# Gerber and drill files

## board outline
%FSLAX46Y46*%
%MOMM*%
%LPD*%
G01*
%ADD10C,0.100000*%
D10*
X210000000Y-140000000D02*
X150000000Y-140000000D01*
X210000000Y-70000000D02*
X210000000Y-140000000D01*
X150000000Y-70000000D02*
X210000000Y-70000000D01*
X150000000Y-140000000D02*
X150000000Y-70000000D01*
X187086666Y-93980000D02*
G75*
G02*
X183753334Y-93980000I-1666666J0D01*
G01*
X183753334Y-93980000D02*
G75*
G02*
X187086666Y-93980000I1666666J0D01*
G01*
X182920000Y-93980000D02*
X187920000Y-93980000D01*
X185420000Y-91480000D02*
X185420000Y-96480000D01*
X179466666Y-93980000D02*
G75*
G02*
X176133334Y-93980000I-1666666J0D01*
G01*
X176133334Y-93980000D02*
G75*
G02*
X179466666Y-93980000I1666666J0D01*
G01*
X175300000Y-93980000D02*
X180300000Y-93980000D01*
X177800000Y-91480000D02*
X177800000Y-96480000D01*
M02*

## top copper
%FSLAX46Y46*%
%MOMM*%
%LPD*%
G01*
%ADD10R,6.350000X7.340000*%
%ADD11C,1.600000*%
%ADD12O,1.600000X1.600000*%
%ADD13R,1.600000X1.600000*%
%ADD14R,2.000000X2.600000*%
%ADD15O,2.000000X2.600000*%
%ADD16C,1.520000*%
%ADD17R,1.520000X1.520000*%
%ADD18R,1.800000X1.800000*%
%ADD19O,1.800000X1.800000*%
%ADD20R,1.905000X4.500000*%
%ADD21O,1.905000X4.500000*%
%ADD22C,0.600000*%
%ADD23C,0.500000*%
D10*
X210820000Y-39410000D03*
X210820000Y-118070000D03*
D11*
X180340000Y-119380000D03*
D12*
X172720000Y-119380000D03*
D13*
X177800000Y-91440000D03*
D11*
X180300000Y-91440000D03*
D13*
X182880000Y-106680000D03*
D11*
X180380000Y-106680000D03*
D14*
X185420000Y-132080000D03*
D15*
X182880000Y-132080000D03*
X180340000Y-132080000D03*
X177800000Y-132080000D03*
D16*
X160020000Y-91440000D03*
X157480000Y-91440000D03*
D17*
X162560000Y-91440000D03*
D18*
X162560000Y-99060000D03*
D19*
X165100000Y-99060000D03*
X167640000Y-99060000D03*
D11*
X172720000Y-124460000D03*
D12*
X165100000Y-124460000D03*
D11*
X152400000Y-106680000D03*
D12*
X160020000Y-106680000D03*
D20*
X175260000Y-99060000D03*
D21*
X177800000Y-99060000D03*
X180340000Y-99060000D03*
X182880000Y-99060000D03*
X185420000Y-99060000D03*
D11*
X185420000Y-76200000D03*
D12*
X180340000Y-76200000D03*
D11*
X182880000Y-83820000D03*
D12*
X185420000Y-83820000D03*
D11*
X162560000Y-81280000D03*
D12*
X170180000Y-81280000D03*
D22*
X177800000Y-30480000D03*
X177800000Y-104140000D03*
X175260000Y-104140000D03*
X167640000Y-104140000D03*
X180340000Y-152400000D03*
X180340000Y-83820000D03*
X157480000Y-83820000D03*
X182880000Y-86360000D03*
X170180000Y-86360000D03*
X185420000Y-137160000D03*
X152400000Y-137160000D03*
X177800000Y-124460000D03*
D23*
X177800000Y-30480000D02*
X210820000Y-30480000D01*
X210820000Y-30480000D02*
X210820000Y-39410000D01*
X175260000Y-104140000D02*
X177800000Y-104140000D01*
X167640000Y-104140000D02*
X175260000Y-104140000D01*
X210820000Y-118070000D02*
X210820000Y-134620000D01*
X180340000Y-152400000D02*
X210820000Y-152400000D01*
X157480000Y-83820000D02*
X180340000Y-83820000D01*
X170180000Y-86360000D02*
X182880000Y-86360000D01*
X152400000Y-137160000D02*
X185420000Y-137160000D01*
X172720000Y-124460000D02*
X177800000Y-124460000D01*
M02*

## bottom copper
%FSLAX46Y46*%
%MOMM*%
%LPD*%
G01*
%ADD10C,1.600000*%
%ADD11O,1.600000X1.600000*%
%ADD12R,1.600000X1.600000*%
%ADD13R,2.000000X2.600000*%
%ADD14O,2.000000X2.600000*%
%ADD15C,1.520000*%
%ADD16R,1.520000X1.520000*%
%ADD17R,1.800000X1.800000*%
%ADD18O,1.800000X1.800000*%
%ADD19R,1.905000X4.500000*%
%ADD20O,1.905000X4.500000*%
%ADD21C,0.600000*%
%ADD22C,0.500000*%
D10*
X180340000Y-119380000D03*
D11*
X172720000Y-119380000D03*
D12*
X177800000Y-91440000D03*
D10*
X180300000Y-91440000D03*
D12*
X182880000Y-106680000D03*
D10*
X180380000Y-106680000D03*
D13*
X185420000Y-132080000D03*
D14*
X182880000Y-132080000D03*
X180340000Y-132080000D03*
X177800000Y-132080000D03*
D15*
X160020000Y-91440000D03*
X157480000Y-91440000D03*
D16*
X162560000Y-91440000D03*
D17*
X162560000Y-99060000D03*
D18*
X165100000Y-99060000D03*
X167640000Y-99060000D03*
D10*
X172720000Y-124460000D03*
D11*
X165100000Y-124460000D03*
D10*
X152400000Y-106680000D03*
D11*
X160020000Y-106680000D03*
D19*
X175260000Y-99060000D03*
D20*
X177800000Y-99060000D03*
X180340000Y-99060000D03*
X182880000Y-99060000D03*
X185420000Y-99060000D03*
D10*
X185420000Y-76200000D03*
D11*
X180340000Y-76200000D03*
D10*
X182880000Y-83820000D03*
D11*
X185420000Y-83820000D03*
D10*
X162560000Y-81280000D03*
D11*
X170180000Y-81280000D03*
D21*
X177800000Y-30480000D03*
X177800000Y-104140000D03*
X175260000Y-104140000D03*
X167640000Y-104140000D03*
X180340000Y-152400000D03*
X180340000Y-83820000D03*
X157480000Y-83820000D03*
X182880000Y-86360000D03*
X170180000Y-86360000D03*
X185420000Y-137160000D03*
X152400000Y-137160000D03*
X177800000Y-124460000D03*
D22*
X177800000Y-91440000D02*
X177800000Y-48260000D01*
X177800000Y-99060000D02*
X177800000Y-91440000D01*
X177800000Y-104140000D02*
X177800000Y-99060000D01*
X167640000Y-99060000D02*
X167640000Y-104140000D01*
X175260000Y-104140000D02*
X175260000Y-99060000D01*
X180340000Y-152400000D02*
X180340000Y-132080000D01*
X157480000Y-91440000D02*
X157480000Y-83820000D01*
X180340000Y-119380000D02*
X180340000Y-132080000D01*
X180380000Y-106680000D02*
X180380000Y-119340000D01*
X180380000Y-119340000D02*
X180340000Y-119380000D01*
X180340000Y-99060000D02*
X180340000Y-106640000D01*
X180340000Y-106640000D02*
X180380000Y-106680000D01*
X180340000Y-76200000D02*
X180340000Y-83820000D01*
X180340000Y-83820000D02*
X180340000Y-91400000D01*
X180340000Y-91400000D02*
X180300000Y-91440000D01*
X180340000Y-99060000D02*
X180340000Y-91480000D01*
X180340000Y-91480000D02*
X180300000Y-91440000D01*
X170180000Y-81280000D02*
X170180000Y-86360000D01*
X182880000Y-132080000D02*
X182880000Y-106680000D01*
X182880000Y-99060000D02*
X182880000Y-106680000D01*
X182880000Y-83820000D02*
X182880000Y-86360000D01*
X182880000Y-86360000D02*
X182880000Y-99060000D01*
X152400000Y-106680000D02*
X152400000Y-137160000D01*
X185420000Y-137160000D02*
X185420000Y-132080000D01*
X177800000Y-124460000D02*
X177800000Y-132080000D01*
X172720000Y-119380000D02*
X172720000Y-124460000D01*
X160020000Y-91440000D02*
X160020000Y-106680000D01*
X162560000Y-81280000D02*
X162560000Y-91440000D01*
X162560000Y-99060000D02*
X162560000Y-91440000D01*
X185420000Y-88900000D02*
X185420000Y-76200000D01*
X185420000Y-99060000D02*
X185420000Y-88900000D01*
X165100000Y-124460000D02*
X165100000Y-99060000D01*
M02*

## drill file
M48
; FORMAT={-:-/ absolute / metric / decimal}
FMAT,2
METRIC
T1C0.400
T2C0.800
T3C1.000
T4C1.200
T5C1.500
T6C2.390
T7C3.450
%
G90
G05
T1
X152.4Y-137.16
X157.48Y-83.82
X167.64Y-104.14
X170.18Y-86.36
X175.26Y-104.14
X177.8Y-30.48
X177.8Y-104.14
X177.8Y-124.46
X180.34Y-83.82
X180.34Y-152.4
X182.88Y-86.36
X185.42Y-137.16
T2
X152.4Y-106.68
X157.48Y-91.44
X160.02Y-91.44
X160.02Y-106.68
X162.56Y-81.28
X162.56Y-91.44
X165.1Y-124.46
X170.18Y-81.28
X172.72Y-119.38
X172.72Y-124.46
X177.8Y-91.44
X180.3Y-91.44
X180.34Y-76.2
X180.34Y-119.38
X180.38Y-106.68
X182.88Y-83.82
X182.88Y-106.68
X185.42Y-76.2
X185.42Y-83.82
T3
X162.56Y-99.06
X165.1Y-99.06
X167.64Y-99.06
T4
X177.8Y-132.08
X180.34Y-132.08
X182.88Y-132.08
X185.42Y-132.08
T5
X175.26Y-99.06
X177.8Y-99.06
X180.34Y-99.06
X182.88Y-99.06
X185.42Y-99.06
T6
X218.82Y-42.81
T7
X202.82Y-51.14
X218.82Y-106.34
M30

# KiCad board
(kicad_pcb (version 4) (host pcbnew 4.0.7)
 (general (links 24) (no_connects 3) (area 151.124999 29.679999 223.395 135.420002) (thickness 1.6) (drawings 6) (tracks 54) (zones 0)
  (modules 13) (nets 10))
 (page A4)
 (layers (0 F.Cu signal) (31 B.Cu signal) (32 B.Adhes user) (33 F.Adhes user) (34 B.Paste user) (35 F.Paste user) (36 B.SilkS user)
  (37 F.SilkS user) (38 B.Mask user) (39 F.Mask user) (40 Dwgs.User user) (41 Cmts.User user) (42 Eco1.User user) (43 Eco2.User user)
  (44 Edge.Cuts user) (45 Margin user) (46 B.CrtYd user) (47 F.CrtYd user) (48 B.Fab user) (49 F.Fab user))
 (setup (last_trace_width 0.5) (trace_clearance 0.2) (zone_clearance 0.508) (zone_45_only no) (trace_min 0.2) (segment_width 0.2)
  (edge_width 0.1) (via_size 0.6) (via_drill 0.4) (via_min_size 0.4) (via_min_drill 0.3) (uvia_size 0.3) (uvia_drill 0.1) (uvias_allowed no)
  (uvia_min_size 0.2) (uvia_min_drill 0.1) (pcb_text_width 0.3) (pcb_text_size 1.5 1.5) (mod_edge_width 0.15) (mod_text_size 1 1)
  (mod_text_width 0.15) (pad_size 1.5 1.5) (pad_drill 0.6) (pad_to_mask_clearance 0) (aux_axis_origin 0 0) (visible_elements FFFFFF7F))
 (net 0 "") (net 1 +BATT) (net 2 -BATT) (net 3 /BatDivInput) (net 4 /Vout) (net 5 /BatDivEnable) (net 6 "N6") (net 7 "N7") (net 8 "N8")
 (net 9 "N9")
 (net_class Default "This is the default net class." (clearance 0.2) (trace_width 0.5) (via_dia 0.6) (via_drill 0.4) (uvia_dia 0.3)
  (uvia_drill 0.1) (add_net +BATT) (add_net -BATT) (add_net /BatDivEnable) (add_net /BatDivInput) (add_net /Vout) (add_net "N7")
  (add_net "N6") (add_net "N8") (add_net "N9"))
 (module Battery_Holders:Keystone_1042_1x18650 (layer F.Cu) (at 210.82 78.74 270)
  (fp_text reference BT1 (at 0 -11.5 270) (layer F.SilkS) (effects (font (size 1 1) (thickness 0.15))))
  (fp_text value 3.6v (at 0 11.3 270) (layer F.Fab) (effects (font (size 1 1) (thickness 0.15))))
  (pad 1 smd rect (at -39.33 0 270) (size 7.34 6.35) (layers F.Cu F.Paste F.Mask) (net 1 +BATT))
  (pad 2 smd rect (at 39.33 0 270) (size 7.34 6.35) (layers F.Cu F.Paste F.Mask) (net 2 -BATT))
  (pad "" np_thru_hole circle (at 27.6 -8 270) (size 3.45 3.45) (drill 3.45) (layers *.Cu *.Mask))
  (pad "" np_thru_hole circle (at -27.6 8 270) (size 3.45 3.45) (drill 3.45) (layers *.Cu *.Mask))
  (pad "" np_thru_hole circle (at -35.93 -8 270) (size 2.39 2.39) (drill 2.39) (layers *.Cu *.Mask)))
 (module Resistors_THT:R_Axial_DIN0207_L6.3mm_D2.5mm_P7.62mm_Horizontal (layer F.Cu) (at 180.34 119.38 180)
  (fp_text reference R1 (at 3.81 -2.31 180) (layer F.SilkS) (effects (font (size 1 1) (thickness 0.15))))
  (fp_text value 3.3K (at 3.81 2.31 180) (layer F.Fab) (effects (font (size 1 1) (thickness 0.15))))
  (pad 1 thru_hole circle (at 0 0 180) (size 1.6 1.6) (drill 0.8) (layers *.Cu *.Mask) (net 2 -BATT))
  (pad 2 thru_hole oval (at 7.62 0 180) (size 1.6 1.6) (drill 0.8) (layers *.Cu *.Mask) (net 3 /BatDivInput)))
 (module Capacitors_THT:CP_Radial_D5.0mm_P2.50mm (layer F.Cu) (at 177.8 91.44)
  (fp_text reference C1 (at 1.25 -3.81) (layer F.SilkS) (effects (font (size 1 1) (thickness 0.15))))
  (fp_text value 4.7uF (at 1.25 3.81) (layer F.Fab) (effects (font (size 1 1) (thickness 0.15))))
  (pad 1 thru_hole rect (at 0 0) (size 1.6 1.6) (drill 0.8) (layers *.Cu *.Mask) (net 1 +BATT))
  (pad 2 thru_hole circle (at 2.5 0) (size 1.6 1.6) (drill 0.8) (layers *.Cu *.Mask) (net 2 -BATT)))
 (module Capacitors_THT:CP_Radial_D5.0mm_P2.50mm (layer F.Cu) (at 182.88 106.68 180)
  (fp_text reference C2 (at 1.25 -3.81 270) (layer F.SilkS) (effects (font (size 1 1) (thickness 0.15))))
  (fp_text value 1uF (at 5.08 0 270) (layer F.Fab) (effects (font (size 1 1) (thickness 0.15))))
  (pad 1 thru_hole rect (at 0 0 180) (size 1.6 1.6) (drill 0.8) (layers *.Cu *.Mask) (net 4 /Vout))
  (pad 2 thru_hole circle (at 2.5 0 180) (size 1.6 1.6) (drill 0.8) (layers *.Cu *.Mask) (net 2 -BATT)))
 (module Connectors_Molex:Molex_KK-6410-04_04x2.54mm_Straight (layer F.Cu) (at 185.42 132.08 180)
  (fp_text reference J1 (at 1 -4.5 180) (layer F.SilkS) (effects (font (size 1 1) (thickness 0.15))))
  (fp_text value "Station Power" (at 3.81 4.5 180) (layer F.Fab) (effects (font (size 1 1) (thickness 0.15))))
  (pad 1 thru_hole rect (at 0 0 180) (size 2 2.6) (drill 1.2) (layers *.Cu *.Mask) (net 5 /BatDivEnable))
  (pad 2 thru_hole oval (at 2.54 0 180) (size 2 2.6) (drill 1.2) (layers *.Cu *.Mask) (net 4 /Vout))
  (pad 3 thru_hole oval (at 5.08 0 180) (size 2 2.6) (drill 1.2) (layers *.Cu *.Mask) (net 2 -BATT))
  (pad 4 thru_hole oval (at 7.62 0 180) (size 2 2.6) (drill 1.2) (layers *.Cu *.Mask) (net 3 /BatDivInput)))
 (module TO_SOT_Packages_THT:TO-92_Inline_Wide (layer F.Cu) (at 162.56 91.44 180)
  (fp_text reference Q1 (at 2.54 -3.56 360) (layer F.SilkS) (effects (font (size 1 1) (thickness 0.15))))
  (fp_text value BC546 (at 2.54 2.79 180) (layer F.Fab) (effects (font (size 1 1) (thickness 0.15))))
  (pad 2 thru_hole circle (at 2.54 0 270) (size 1.52 1.52) (drill 0.8) (layers *.Cu *.Mask) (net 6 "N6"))
  (pad 3 thru_hole circle (at 5.08 0 270) (size 1.52 1.52) (drill 0.8) (layers *.Cu *.Mask) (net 2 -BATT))
  (pad 1 thru_hole rect (at 0 0 270) (size 1.52 1.52) (drill 0.8) (layers *.Cu *.Mask) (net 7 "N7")))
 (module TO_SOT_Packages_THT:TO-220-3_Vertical (layer F.Cu) (at 162.56 99.06)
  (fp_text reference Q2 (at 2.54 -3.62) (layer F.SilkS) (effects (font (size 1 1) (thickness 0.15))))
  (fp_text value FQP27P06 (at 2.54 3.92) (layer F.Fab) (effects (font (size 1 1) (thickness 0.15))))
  (pad 1 thru_hole rect (at 0 0) (size 1.8 1.8) (drill 1) (layers *.Cu *.Mask) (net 7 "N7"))
  (pad 2 thru_hole oval (at 2.54 0) (size 1.8 1.8) (drill 1) (layers *.Cu *.Mask) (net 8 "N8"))
  (pad 3 thru_hole oval (at 5.08 0) (size 1.8 1.8) (drill 1) (layers *.Cu *.Mask) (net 1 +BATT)))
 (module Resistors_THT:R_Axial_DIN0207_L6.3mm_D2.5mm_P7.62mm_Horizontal (layer F.Cu) (at 172.72 124.46 180)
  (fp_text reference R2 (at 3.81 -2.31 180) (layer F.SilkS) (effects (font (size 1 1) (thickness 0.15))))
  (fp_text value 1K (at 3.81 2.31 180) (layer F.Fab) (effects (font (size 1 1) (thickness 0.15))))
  (pad 1 thru_hole circle (at 0 0 180) (size 1.6 1.6) (drill 0.8) (layers *.Cu *.Mask) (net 3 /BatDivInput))
  (pad 2 thru_hole oval (at 7.62 0 180) (size 1.6 1.6) (drill 0.8) (layers *.Cu *.Mask) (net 8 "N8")))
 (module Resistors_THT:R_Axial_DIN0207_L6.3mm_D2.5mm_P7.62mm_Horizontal (layer F.Cu) (at 152.4 106.68)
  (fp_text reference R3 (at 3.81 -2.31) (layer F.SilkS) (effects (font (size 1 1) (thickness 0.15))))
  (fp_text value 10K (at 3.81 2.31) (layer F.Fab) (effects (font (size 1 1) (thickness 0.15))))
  (pad 1 thru_hole circle (at 0 0) (size 1.6 1.6) (drill 0.8) (layers *.Cu *.Mask) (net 5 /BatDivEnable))
  (pad 2 thru_hole oval (at 7.62 0) (size 1.6 1.6) (drill 0.8) (layers *.Cu *.Mask) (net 6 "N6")))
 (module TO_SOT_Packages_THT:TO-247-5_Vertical (layer F.Cu) (at 175.26 99.06)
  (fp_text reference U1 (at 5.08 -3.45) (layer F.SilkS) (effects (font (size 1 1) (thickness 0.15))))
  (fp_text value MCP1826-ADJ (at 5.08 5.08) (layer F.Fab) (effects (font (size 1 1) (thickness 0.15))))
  (pad 1 thru_hole rect (at 0 0) (size 1.905 4.5) (drill 1.5) (layers *.Cu *.Mask) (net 1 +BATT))
  (pad 2 thru_hole oval (at 2.54 0) (size 1.905 4.5) (drill 1.5) (layers *.Cu *.Mask) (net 1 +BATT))
  (pad 3 thru_hole oval (at 5.08 0) (size 1.905 4.5) (drill 1.5) (layers *.Cu *.Mask) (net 2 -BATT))
  (pad 4 thru_hole oval (at 7.62 0) (size 1.905 4.5) (drill 1.5) (layers *.Cu *.Mask) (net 4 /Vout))
  (pad 5 thru_hole oval (at 10.16 0) (size 1.905 4.5) (drill 1.5) (layers *.Cu *.Mask) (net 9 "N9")))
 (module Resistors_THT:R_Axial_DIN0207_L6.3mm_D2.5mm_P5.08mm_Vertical (layer F.Cu) (at 185.42 76.2 180)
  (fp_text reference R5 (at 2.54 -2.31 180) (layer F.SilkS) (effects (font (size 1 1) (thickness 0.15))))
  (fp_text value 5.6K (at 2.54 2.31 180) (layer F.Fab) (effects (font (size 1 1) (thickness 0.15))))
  (pad 1 thru_hole circle (at 0 0 180) (size 1.6 1.6) (drill 0.8) (layers *.Cu *.Mask) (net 9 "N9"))
  (pad 2 thru_hole oval (at 5.08 0 180) (size 1.6 1.6) (drill 0.8) (layers *.Cu *.Mask) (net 2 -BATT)))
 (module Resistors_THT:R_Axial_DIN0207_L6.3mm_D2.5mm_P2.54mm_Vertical (layer F.Cu) (at 182.88 83.82)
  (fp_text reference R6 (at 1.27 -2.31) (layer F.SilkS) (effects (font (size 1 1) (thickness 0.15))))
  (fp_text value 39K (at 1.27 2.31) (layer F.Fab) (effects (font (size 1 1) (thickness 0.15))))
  (pad 1 thru_hole circle (at 0 0) (size 1.6 1.6) (drill 0.8) (layers *.Cu *.Mask) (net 4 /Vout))
  (pad 2 thru_hole oval (at 2.54 0) (size 1.6 1.6) (drill 0.8) (layers *.Cu *.Mask) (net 9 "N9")))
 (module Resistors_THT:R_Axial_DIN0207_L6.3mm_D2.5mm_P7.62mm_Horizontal (layer F.Cu) (at 162.56 81.28)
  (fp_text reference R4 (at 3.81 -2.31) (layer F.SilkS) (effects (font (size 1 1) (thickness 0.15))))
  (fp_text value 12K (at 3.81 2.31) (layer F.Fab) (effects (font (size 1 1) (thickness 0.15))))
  (pad 1 thru_hole circle (at 0 0) (size 1.6 1.6) (drill 0.8) (layers *.Cu *.Mask) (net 7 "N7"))
  (pad 2 thru_hole oval (at 7.62 0) (size 1.6 1.6) (drill 0.8) (layers *.Cu *.Mask) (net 4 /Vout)))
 (gr_line (start 210 140) (end 150 140) (angle 90) (layer Edge.Cuts) (width 0.1))
 (gr_line (start 210 70) (end 210 140) (angle 90) (layer Edge.Cuts) (width 0.1))
 (gr_line (start 150 70) (end 210 70) (angle 90) (layer Edge.Cuts) (width 0.1))
 (gr_line (start 150 140) (end 150 70) (angle 90) (layer Edge.Cuts) (width 0.1))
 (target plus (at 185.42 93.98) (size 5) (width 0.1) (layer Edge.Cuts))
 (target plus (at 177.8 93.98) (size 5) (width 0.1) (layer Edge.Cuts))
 (segment (start 177.8 30.48) (end 210.82 30.48) (width 0.5) (layer F.Cu) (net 1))
 (via (at 177.8 30.48) (size 0.6) (drill 0.4) (layers F.Cu B.Cu) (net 1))
 (segment (start 177.8 91.44) (end 177.8 48.26) (width 0.5) (layer B.Cu) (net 1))
 (segment (start 210.82 30.48) (end 210.82 39.41) (width 0.5) (layer F.Cu) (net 1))
 (segment (start 177.8 99.06) (end 177.8 91.44) (width 0.5) (layer B.Cu) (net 1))
 (segment (start 175.26 104.14) (end 177.8 104.14) (width 0.5) (layer F.Cu) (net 1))
 (segment (start 177.8 104.14) (end 177.8 99.06) (width 0.5) (layer B.Cu) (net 1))
 (via (at 177.8 104.14) (size 0.6) (drill 0.4) (layers F.Cu B.Cu) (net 1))
 (segment (start 167.64 99.06) (end 167.64 104.14) (width 0.5) (layer B.Cu) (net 1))
 (segment (start 175.26 104.14) (end 175.26 99.06) (width 0.5) (layer B.Cu) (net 1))
 (via (at 175.26 104.14) (size 0.6) (drill 0.4) (layers F.Cu B.Cu) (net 1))
 (segment (start 167.64 104.14) (end 175.26 104.14) (width 0.5) (layer F.Cu) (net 1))
 (via (at 167.64 104.14) (size 0.6) (drill 0.4) (layers F.Cu B.Cu) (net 1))
 (segment (start 210.82 118.07) (end 210.82 134.62) (width 0.5) (layer F.Cu) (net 2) (status 10))
 (via (at 180.34 152.4) (size 0.6) (drill 0.4) (layers F.Cu B.Cu) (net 2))
 (segment (start 180.34 152.4) (end 210.82 152.4) (width 0.5) (layer F.Cu) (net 2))
 (segment (start 180.34 152.4) (end 180.34 132.08) (width 0.5) (layer B.Cu) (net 2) (status 20))
 (segment (start 157.48 91.44) (end 157.48 83.82) (width 0.5) (layer B.Cu) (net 2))
 (via (at 180.34 83.82) (size 0.6) (drill 0.4) (layers F.Cu B.Cu) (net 2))
 (segment (start 157.48 83.82) (end 180.34 83.82) (width 0.5) (layer F.Cu) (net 2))
 (via (at 157.48 83.82) (size 0.6) (drill 0.4) (layers F.Cu B.Cu) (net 2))
 (segment (start 180.34 119.38) (end 180.34 132.08) (width 0.5) (layer B.Cu) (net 2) (status 20))
 (segment (start 180.38 106.68) (end 180.38 119.34) (width 0.5) (layer B.Cu) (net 2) (status 20))
 (segment (start 180.38 119.34) (end 180.34 119.38) (width 0.5) (layer B.Cu) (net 2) (status 30))
 (segment (start 180.34 99.06) (end 180.34 106.64) (width 0.5) (layer B.Cu) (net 2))
 (segment (start 180.34 106.64) (end 180.38 106.68) (width 0.5) (layer B.Cu) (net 2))
 (segment (start 180.34 76.2) (end 180.34 83.82) (width 0.5) (layer B.Cu) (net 2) (status 10))
 (segment (start 180.34 83.82) (end 180.34 91.4) (width 0.5) (layer B.Cu) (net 2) (status 20))
 (segment (start 180.34 91.4) (end 180.3 91.44) (width 0.5) (layer B.Cu) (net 2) (status 30))
 (segment (start 180.34 99.06) (end 180.34 91.48) (width 0.5) (layer B.Cu) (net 2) (status 20))
 (segment (start 180.34 91.48) (end 180.3 91.44) (width 0.5) (layer B.Cu) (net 2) (status 30))
 (segment (start 170.18 81.28) (end 170.18 86.36) (width 0.5) (layer B.Cu) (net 4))
 (via (at 182.88 86.36) (size 0.6) (drill 0.4) (layers F.Cu B.Cu) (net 4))
 (segment (start 170.18 86.36) (end 182.88 86.36) (width 0.5) (layer F.Cu) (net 4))
 (via (at 170.18 86.36) (size 0.6) (drill 0.4) (layers F.Cu B.Cu) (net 4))
 (segment (start 182.88 132.08) (end 182.88 106.68) (width 0.5) (layer B.Cu) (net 4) (status 10))
 (segment (start 182.88 99.06) (end 182.88 106.68) (width 0.5) (layer B.Cu) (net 4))
 (segment (start 182.88 83.82) (end 182.88 86.36) (width 0.5) (layer B.Cu) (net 4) (status 10))
 (segment (start 182.88 86.36) (end 182.88 99.06) (width 0.5) (layer B.Cu) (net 4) (status 10))
 (segment (start 152.4 106.68) (end 152.4 137.16) (width 0.5) (layer B.Cu) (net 5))
 (segment (start 185.42 137.16) (end 185.42 132.08) (width 0.5) (layer B.Cu) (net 5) (status 20))
 (via (at 185.42 137.16) (size 0.6) (drill 0.4) (layers F.Cu B.Cu) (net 5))
 (segment (start 152.4 137.16) (end 185.42 137.16) (width 0.5) (layer F.Cu) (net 5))
 (via (at 152.4 137.16) (size 0.6) (drill 0.4) (layers F.Cu B.Cu) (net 5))
 (segment (start 172.72 124.46) (end 177.8 124.46) (width 0.5) (layer F.Cu) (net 3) (status 10))
 (segment (start 177.8 124.46) (end 177.8 132.08) (width 0.5) (layer B.Cu) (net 3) (status 20))
 (via (at 177.8 124.46) (size 0.6) (drill 0.4) (layers F.Cu B.Cu) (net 3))
 (segment (start 172.72 119.38) (end 172.72 124.46) (width 0.5) (layer B.Cu) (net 3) (status 10))
 (segment (start 160.02 91.44) (end 160.02 106.68) (width 0.5) (layer B.Cu) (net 6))
 (segment (start 162.56 81.28) (end 162.56 91.44) (width 0.5) (layer B.Cu) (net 7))
 (segment (start 162.56 99.06) (end 162.56 91.44) (width 0.5) (layer B.Cu) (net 7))
 (segment (start 185.42 88.9) (end 185.42 76.2) (width 0.5) (layer B.Cu) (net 9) (status 20))
 (segment (start 185.42 99.06) (end 185.42 88.9) (width 0.5) (layer B.Cu) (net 9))
 (segment (start 165.1 124.46) (end 165.1 99.06) (width 0.5) (layer B.Cu) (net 8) (status 10)))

